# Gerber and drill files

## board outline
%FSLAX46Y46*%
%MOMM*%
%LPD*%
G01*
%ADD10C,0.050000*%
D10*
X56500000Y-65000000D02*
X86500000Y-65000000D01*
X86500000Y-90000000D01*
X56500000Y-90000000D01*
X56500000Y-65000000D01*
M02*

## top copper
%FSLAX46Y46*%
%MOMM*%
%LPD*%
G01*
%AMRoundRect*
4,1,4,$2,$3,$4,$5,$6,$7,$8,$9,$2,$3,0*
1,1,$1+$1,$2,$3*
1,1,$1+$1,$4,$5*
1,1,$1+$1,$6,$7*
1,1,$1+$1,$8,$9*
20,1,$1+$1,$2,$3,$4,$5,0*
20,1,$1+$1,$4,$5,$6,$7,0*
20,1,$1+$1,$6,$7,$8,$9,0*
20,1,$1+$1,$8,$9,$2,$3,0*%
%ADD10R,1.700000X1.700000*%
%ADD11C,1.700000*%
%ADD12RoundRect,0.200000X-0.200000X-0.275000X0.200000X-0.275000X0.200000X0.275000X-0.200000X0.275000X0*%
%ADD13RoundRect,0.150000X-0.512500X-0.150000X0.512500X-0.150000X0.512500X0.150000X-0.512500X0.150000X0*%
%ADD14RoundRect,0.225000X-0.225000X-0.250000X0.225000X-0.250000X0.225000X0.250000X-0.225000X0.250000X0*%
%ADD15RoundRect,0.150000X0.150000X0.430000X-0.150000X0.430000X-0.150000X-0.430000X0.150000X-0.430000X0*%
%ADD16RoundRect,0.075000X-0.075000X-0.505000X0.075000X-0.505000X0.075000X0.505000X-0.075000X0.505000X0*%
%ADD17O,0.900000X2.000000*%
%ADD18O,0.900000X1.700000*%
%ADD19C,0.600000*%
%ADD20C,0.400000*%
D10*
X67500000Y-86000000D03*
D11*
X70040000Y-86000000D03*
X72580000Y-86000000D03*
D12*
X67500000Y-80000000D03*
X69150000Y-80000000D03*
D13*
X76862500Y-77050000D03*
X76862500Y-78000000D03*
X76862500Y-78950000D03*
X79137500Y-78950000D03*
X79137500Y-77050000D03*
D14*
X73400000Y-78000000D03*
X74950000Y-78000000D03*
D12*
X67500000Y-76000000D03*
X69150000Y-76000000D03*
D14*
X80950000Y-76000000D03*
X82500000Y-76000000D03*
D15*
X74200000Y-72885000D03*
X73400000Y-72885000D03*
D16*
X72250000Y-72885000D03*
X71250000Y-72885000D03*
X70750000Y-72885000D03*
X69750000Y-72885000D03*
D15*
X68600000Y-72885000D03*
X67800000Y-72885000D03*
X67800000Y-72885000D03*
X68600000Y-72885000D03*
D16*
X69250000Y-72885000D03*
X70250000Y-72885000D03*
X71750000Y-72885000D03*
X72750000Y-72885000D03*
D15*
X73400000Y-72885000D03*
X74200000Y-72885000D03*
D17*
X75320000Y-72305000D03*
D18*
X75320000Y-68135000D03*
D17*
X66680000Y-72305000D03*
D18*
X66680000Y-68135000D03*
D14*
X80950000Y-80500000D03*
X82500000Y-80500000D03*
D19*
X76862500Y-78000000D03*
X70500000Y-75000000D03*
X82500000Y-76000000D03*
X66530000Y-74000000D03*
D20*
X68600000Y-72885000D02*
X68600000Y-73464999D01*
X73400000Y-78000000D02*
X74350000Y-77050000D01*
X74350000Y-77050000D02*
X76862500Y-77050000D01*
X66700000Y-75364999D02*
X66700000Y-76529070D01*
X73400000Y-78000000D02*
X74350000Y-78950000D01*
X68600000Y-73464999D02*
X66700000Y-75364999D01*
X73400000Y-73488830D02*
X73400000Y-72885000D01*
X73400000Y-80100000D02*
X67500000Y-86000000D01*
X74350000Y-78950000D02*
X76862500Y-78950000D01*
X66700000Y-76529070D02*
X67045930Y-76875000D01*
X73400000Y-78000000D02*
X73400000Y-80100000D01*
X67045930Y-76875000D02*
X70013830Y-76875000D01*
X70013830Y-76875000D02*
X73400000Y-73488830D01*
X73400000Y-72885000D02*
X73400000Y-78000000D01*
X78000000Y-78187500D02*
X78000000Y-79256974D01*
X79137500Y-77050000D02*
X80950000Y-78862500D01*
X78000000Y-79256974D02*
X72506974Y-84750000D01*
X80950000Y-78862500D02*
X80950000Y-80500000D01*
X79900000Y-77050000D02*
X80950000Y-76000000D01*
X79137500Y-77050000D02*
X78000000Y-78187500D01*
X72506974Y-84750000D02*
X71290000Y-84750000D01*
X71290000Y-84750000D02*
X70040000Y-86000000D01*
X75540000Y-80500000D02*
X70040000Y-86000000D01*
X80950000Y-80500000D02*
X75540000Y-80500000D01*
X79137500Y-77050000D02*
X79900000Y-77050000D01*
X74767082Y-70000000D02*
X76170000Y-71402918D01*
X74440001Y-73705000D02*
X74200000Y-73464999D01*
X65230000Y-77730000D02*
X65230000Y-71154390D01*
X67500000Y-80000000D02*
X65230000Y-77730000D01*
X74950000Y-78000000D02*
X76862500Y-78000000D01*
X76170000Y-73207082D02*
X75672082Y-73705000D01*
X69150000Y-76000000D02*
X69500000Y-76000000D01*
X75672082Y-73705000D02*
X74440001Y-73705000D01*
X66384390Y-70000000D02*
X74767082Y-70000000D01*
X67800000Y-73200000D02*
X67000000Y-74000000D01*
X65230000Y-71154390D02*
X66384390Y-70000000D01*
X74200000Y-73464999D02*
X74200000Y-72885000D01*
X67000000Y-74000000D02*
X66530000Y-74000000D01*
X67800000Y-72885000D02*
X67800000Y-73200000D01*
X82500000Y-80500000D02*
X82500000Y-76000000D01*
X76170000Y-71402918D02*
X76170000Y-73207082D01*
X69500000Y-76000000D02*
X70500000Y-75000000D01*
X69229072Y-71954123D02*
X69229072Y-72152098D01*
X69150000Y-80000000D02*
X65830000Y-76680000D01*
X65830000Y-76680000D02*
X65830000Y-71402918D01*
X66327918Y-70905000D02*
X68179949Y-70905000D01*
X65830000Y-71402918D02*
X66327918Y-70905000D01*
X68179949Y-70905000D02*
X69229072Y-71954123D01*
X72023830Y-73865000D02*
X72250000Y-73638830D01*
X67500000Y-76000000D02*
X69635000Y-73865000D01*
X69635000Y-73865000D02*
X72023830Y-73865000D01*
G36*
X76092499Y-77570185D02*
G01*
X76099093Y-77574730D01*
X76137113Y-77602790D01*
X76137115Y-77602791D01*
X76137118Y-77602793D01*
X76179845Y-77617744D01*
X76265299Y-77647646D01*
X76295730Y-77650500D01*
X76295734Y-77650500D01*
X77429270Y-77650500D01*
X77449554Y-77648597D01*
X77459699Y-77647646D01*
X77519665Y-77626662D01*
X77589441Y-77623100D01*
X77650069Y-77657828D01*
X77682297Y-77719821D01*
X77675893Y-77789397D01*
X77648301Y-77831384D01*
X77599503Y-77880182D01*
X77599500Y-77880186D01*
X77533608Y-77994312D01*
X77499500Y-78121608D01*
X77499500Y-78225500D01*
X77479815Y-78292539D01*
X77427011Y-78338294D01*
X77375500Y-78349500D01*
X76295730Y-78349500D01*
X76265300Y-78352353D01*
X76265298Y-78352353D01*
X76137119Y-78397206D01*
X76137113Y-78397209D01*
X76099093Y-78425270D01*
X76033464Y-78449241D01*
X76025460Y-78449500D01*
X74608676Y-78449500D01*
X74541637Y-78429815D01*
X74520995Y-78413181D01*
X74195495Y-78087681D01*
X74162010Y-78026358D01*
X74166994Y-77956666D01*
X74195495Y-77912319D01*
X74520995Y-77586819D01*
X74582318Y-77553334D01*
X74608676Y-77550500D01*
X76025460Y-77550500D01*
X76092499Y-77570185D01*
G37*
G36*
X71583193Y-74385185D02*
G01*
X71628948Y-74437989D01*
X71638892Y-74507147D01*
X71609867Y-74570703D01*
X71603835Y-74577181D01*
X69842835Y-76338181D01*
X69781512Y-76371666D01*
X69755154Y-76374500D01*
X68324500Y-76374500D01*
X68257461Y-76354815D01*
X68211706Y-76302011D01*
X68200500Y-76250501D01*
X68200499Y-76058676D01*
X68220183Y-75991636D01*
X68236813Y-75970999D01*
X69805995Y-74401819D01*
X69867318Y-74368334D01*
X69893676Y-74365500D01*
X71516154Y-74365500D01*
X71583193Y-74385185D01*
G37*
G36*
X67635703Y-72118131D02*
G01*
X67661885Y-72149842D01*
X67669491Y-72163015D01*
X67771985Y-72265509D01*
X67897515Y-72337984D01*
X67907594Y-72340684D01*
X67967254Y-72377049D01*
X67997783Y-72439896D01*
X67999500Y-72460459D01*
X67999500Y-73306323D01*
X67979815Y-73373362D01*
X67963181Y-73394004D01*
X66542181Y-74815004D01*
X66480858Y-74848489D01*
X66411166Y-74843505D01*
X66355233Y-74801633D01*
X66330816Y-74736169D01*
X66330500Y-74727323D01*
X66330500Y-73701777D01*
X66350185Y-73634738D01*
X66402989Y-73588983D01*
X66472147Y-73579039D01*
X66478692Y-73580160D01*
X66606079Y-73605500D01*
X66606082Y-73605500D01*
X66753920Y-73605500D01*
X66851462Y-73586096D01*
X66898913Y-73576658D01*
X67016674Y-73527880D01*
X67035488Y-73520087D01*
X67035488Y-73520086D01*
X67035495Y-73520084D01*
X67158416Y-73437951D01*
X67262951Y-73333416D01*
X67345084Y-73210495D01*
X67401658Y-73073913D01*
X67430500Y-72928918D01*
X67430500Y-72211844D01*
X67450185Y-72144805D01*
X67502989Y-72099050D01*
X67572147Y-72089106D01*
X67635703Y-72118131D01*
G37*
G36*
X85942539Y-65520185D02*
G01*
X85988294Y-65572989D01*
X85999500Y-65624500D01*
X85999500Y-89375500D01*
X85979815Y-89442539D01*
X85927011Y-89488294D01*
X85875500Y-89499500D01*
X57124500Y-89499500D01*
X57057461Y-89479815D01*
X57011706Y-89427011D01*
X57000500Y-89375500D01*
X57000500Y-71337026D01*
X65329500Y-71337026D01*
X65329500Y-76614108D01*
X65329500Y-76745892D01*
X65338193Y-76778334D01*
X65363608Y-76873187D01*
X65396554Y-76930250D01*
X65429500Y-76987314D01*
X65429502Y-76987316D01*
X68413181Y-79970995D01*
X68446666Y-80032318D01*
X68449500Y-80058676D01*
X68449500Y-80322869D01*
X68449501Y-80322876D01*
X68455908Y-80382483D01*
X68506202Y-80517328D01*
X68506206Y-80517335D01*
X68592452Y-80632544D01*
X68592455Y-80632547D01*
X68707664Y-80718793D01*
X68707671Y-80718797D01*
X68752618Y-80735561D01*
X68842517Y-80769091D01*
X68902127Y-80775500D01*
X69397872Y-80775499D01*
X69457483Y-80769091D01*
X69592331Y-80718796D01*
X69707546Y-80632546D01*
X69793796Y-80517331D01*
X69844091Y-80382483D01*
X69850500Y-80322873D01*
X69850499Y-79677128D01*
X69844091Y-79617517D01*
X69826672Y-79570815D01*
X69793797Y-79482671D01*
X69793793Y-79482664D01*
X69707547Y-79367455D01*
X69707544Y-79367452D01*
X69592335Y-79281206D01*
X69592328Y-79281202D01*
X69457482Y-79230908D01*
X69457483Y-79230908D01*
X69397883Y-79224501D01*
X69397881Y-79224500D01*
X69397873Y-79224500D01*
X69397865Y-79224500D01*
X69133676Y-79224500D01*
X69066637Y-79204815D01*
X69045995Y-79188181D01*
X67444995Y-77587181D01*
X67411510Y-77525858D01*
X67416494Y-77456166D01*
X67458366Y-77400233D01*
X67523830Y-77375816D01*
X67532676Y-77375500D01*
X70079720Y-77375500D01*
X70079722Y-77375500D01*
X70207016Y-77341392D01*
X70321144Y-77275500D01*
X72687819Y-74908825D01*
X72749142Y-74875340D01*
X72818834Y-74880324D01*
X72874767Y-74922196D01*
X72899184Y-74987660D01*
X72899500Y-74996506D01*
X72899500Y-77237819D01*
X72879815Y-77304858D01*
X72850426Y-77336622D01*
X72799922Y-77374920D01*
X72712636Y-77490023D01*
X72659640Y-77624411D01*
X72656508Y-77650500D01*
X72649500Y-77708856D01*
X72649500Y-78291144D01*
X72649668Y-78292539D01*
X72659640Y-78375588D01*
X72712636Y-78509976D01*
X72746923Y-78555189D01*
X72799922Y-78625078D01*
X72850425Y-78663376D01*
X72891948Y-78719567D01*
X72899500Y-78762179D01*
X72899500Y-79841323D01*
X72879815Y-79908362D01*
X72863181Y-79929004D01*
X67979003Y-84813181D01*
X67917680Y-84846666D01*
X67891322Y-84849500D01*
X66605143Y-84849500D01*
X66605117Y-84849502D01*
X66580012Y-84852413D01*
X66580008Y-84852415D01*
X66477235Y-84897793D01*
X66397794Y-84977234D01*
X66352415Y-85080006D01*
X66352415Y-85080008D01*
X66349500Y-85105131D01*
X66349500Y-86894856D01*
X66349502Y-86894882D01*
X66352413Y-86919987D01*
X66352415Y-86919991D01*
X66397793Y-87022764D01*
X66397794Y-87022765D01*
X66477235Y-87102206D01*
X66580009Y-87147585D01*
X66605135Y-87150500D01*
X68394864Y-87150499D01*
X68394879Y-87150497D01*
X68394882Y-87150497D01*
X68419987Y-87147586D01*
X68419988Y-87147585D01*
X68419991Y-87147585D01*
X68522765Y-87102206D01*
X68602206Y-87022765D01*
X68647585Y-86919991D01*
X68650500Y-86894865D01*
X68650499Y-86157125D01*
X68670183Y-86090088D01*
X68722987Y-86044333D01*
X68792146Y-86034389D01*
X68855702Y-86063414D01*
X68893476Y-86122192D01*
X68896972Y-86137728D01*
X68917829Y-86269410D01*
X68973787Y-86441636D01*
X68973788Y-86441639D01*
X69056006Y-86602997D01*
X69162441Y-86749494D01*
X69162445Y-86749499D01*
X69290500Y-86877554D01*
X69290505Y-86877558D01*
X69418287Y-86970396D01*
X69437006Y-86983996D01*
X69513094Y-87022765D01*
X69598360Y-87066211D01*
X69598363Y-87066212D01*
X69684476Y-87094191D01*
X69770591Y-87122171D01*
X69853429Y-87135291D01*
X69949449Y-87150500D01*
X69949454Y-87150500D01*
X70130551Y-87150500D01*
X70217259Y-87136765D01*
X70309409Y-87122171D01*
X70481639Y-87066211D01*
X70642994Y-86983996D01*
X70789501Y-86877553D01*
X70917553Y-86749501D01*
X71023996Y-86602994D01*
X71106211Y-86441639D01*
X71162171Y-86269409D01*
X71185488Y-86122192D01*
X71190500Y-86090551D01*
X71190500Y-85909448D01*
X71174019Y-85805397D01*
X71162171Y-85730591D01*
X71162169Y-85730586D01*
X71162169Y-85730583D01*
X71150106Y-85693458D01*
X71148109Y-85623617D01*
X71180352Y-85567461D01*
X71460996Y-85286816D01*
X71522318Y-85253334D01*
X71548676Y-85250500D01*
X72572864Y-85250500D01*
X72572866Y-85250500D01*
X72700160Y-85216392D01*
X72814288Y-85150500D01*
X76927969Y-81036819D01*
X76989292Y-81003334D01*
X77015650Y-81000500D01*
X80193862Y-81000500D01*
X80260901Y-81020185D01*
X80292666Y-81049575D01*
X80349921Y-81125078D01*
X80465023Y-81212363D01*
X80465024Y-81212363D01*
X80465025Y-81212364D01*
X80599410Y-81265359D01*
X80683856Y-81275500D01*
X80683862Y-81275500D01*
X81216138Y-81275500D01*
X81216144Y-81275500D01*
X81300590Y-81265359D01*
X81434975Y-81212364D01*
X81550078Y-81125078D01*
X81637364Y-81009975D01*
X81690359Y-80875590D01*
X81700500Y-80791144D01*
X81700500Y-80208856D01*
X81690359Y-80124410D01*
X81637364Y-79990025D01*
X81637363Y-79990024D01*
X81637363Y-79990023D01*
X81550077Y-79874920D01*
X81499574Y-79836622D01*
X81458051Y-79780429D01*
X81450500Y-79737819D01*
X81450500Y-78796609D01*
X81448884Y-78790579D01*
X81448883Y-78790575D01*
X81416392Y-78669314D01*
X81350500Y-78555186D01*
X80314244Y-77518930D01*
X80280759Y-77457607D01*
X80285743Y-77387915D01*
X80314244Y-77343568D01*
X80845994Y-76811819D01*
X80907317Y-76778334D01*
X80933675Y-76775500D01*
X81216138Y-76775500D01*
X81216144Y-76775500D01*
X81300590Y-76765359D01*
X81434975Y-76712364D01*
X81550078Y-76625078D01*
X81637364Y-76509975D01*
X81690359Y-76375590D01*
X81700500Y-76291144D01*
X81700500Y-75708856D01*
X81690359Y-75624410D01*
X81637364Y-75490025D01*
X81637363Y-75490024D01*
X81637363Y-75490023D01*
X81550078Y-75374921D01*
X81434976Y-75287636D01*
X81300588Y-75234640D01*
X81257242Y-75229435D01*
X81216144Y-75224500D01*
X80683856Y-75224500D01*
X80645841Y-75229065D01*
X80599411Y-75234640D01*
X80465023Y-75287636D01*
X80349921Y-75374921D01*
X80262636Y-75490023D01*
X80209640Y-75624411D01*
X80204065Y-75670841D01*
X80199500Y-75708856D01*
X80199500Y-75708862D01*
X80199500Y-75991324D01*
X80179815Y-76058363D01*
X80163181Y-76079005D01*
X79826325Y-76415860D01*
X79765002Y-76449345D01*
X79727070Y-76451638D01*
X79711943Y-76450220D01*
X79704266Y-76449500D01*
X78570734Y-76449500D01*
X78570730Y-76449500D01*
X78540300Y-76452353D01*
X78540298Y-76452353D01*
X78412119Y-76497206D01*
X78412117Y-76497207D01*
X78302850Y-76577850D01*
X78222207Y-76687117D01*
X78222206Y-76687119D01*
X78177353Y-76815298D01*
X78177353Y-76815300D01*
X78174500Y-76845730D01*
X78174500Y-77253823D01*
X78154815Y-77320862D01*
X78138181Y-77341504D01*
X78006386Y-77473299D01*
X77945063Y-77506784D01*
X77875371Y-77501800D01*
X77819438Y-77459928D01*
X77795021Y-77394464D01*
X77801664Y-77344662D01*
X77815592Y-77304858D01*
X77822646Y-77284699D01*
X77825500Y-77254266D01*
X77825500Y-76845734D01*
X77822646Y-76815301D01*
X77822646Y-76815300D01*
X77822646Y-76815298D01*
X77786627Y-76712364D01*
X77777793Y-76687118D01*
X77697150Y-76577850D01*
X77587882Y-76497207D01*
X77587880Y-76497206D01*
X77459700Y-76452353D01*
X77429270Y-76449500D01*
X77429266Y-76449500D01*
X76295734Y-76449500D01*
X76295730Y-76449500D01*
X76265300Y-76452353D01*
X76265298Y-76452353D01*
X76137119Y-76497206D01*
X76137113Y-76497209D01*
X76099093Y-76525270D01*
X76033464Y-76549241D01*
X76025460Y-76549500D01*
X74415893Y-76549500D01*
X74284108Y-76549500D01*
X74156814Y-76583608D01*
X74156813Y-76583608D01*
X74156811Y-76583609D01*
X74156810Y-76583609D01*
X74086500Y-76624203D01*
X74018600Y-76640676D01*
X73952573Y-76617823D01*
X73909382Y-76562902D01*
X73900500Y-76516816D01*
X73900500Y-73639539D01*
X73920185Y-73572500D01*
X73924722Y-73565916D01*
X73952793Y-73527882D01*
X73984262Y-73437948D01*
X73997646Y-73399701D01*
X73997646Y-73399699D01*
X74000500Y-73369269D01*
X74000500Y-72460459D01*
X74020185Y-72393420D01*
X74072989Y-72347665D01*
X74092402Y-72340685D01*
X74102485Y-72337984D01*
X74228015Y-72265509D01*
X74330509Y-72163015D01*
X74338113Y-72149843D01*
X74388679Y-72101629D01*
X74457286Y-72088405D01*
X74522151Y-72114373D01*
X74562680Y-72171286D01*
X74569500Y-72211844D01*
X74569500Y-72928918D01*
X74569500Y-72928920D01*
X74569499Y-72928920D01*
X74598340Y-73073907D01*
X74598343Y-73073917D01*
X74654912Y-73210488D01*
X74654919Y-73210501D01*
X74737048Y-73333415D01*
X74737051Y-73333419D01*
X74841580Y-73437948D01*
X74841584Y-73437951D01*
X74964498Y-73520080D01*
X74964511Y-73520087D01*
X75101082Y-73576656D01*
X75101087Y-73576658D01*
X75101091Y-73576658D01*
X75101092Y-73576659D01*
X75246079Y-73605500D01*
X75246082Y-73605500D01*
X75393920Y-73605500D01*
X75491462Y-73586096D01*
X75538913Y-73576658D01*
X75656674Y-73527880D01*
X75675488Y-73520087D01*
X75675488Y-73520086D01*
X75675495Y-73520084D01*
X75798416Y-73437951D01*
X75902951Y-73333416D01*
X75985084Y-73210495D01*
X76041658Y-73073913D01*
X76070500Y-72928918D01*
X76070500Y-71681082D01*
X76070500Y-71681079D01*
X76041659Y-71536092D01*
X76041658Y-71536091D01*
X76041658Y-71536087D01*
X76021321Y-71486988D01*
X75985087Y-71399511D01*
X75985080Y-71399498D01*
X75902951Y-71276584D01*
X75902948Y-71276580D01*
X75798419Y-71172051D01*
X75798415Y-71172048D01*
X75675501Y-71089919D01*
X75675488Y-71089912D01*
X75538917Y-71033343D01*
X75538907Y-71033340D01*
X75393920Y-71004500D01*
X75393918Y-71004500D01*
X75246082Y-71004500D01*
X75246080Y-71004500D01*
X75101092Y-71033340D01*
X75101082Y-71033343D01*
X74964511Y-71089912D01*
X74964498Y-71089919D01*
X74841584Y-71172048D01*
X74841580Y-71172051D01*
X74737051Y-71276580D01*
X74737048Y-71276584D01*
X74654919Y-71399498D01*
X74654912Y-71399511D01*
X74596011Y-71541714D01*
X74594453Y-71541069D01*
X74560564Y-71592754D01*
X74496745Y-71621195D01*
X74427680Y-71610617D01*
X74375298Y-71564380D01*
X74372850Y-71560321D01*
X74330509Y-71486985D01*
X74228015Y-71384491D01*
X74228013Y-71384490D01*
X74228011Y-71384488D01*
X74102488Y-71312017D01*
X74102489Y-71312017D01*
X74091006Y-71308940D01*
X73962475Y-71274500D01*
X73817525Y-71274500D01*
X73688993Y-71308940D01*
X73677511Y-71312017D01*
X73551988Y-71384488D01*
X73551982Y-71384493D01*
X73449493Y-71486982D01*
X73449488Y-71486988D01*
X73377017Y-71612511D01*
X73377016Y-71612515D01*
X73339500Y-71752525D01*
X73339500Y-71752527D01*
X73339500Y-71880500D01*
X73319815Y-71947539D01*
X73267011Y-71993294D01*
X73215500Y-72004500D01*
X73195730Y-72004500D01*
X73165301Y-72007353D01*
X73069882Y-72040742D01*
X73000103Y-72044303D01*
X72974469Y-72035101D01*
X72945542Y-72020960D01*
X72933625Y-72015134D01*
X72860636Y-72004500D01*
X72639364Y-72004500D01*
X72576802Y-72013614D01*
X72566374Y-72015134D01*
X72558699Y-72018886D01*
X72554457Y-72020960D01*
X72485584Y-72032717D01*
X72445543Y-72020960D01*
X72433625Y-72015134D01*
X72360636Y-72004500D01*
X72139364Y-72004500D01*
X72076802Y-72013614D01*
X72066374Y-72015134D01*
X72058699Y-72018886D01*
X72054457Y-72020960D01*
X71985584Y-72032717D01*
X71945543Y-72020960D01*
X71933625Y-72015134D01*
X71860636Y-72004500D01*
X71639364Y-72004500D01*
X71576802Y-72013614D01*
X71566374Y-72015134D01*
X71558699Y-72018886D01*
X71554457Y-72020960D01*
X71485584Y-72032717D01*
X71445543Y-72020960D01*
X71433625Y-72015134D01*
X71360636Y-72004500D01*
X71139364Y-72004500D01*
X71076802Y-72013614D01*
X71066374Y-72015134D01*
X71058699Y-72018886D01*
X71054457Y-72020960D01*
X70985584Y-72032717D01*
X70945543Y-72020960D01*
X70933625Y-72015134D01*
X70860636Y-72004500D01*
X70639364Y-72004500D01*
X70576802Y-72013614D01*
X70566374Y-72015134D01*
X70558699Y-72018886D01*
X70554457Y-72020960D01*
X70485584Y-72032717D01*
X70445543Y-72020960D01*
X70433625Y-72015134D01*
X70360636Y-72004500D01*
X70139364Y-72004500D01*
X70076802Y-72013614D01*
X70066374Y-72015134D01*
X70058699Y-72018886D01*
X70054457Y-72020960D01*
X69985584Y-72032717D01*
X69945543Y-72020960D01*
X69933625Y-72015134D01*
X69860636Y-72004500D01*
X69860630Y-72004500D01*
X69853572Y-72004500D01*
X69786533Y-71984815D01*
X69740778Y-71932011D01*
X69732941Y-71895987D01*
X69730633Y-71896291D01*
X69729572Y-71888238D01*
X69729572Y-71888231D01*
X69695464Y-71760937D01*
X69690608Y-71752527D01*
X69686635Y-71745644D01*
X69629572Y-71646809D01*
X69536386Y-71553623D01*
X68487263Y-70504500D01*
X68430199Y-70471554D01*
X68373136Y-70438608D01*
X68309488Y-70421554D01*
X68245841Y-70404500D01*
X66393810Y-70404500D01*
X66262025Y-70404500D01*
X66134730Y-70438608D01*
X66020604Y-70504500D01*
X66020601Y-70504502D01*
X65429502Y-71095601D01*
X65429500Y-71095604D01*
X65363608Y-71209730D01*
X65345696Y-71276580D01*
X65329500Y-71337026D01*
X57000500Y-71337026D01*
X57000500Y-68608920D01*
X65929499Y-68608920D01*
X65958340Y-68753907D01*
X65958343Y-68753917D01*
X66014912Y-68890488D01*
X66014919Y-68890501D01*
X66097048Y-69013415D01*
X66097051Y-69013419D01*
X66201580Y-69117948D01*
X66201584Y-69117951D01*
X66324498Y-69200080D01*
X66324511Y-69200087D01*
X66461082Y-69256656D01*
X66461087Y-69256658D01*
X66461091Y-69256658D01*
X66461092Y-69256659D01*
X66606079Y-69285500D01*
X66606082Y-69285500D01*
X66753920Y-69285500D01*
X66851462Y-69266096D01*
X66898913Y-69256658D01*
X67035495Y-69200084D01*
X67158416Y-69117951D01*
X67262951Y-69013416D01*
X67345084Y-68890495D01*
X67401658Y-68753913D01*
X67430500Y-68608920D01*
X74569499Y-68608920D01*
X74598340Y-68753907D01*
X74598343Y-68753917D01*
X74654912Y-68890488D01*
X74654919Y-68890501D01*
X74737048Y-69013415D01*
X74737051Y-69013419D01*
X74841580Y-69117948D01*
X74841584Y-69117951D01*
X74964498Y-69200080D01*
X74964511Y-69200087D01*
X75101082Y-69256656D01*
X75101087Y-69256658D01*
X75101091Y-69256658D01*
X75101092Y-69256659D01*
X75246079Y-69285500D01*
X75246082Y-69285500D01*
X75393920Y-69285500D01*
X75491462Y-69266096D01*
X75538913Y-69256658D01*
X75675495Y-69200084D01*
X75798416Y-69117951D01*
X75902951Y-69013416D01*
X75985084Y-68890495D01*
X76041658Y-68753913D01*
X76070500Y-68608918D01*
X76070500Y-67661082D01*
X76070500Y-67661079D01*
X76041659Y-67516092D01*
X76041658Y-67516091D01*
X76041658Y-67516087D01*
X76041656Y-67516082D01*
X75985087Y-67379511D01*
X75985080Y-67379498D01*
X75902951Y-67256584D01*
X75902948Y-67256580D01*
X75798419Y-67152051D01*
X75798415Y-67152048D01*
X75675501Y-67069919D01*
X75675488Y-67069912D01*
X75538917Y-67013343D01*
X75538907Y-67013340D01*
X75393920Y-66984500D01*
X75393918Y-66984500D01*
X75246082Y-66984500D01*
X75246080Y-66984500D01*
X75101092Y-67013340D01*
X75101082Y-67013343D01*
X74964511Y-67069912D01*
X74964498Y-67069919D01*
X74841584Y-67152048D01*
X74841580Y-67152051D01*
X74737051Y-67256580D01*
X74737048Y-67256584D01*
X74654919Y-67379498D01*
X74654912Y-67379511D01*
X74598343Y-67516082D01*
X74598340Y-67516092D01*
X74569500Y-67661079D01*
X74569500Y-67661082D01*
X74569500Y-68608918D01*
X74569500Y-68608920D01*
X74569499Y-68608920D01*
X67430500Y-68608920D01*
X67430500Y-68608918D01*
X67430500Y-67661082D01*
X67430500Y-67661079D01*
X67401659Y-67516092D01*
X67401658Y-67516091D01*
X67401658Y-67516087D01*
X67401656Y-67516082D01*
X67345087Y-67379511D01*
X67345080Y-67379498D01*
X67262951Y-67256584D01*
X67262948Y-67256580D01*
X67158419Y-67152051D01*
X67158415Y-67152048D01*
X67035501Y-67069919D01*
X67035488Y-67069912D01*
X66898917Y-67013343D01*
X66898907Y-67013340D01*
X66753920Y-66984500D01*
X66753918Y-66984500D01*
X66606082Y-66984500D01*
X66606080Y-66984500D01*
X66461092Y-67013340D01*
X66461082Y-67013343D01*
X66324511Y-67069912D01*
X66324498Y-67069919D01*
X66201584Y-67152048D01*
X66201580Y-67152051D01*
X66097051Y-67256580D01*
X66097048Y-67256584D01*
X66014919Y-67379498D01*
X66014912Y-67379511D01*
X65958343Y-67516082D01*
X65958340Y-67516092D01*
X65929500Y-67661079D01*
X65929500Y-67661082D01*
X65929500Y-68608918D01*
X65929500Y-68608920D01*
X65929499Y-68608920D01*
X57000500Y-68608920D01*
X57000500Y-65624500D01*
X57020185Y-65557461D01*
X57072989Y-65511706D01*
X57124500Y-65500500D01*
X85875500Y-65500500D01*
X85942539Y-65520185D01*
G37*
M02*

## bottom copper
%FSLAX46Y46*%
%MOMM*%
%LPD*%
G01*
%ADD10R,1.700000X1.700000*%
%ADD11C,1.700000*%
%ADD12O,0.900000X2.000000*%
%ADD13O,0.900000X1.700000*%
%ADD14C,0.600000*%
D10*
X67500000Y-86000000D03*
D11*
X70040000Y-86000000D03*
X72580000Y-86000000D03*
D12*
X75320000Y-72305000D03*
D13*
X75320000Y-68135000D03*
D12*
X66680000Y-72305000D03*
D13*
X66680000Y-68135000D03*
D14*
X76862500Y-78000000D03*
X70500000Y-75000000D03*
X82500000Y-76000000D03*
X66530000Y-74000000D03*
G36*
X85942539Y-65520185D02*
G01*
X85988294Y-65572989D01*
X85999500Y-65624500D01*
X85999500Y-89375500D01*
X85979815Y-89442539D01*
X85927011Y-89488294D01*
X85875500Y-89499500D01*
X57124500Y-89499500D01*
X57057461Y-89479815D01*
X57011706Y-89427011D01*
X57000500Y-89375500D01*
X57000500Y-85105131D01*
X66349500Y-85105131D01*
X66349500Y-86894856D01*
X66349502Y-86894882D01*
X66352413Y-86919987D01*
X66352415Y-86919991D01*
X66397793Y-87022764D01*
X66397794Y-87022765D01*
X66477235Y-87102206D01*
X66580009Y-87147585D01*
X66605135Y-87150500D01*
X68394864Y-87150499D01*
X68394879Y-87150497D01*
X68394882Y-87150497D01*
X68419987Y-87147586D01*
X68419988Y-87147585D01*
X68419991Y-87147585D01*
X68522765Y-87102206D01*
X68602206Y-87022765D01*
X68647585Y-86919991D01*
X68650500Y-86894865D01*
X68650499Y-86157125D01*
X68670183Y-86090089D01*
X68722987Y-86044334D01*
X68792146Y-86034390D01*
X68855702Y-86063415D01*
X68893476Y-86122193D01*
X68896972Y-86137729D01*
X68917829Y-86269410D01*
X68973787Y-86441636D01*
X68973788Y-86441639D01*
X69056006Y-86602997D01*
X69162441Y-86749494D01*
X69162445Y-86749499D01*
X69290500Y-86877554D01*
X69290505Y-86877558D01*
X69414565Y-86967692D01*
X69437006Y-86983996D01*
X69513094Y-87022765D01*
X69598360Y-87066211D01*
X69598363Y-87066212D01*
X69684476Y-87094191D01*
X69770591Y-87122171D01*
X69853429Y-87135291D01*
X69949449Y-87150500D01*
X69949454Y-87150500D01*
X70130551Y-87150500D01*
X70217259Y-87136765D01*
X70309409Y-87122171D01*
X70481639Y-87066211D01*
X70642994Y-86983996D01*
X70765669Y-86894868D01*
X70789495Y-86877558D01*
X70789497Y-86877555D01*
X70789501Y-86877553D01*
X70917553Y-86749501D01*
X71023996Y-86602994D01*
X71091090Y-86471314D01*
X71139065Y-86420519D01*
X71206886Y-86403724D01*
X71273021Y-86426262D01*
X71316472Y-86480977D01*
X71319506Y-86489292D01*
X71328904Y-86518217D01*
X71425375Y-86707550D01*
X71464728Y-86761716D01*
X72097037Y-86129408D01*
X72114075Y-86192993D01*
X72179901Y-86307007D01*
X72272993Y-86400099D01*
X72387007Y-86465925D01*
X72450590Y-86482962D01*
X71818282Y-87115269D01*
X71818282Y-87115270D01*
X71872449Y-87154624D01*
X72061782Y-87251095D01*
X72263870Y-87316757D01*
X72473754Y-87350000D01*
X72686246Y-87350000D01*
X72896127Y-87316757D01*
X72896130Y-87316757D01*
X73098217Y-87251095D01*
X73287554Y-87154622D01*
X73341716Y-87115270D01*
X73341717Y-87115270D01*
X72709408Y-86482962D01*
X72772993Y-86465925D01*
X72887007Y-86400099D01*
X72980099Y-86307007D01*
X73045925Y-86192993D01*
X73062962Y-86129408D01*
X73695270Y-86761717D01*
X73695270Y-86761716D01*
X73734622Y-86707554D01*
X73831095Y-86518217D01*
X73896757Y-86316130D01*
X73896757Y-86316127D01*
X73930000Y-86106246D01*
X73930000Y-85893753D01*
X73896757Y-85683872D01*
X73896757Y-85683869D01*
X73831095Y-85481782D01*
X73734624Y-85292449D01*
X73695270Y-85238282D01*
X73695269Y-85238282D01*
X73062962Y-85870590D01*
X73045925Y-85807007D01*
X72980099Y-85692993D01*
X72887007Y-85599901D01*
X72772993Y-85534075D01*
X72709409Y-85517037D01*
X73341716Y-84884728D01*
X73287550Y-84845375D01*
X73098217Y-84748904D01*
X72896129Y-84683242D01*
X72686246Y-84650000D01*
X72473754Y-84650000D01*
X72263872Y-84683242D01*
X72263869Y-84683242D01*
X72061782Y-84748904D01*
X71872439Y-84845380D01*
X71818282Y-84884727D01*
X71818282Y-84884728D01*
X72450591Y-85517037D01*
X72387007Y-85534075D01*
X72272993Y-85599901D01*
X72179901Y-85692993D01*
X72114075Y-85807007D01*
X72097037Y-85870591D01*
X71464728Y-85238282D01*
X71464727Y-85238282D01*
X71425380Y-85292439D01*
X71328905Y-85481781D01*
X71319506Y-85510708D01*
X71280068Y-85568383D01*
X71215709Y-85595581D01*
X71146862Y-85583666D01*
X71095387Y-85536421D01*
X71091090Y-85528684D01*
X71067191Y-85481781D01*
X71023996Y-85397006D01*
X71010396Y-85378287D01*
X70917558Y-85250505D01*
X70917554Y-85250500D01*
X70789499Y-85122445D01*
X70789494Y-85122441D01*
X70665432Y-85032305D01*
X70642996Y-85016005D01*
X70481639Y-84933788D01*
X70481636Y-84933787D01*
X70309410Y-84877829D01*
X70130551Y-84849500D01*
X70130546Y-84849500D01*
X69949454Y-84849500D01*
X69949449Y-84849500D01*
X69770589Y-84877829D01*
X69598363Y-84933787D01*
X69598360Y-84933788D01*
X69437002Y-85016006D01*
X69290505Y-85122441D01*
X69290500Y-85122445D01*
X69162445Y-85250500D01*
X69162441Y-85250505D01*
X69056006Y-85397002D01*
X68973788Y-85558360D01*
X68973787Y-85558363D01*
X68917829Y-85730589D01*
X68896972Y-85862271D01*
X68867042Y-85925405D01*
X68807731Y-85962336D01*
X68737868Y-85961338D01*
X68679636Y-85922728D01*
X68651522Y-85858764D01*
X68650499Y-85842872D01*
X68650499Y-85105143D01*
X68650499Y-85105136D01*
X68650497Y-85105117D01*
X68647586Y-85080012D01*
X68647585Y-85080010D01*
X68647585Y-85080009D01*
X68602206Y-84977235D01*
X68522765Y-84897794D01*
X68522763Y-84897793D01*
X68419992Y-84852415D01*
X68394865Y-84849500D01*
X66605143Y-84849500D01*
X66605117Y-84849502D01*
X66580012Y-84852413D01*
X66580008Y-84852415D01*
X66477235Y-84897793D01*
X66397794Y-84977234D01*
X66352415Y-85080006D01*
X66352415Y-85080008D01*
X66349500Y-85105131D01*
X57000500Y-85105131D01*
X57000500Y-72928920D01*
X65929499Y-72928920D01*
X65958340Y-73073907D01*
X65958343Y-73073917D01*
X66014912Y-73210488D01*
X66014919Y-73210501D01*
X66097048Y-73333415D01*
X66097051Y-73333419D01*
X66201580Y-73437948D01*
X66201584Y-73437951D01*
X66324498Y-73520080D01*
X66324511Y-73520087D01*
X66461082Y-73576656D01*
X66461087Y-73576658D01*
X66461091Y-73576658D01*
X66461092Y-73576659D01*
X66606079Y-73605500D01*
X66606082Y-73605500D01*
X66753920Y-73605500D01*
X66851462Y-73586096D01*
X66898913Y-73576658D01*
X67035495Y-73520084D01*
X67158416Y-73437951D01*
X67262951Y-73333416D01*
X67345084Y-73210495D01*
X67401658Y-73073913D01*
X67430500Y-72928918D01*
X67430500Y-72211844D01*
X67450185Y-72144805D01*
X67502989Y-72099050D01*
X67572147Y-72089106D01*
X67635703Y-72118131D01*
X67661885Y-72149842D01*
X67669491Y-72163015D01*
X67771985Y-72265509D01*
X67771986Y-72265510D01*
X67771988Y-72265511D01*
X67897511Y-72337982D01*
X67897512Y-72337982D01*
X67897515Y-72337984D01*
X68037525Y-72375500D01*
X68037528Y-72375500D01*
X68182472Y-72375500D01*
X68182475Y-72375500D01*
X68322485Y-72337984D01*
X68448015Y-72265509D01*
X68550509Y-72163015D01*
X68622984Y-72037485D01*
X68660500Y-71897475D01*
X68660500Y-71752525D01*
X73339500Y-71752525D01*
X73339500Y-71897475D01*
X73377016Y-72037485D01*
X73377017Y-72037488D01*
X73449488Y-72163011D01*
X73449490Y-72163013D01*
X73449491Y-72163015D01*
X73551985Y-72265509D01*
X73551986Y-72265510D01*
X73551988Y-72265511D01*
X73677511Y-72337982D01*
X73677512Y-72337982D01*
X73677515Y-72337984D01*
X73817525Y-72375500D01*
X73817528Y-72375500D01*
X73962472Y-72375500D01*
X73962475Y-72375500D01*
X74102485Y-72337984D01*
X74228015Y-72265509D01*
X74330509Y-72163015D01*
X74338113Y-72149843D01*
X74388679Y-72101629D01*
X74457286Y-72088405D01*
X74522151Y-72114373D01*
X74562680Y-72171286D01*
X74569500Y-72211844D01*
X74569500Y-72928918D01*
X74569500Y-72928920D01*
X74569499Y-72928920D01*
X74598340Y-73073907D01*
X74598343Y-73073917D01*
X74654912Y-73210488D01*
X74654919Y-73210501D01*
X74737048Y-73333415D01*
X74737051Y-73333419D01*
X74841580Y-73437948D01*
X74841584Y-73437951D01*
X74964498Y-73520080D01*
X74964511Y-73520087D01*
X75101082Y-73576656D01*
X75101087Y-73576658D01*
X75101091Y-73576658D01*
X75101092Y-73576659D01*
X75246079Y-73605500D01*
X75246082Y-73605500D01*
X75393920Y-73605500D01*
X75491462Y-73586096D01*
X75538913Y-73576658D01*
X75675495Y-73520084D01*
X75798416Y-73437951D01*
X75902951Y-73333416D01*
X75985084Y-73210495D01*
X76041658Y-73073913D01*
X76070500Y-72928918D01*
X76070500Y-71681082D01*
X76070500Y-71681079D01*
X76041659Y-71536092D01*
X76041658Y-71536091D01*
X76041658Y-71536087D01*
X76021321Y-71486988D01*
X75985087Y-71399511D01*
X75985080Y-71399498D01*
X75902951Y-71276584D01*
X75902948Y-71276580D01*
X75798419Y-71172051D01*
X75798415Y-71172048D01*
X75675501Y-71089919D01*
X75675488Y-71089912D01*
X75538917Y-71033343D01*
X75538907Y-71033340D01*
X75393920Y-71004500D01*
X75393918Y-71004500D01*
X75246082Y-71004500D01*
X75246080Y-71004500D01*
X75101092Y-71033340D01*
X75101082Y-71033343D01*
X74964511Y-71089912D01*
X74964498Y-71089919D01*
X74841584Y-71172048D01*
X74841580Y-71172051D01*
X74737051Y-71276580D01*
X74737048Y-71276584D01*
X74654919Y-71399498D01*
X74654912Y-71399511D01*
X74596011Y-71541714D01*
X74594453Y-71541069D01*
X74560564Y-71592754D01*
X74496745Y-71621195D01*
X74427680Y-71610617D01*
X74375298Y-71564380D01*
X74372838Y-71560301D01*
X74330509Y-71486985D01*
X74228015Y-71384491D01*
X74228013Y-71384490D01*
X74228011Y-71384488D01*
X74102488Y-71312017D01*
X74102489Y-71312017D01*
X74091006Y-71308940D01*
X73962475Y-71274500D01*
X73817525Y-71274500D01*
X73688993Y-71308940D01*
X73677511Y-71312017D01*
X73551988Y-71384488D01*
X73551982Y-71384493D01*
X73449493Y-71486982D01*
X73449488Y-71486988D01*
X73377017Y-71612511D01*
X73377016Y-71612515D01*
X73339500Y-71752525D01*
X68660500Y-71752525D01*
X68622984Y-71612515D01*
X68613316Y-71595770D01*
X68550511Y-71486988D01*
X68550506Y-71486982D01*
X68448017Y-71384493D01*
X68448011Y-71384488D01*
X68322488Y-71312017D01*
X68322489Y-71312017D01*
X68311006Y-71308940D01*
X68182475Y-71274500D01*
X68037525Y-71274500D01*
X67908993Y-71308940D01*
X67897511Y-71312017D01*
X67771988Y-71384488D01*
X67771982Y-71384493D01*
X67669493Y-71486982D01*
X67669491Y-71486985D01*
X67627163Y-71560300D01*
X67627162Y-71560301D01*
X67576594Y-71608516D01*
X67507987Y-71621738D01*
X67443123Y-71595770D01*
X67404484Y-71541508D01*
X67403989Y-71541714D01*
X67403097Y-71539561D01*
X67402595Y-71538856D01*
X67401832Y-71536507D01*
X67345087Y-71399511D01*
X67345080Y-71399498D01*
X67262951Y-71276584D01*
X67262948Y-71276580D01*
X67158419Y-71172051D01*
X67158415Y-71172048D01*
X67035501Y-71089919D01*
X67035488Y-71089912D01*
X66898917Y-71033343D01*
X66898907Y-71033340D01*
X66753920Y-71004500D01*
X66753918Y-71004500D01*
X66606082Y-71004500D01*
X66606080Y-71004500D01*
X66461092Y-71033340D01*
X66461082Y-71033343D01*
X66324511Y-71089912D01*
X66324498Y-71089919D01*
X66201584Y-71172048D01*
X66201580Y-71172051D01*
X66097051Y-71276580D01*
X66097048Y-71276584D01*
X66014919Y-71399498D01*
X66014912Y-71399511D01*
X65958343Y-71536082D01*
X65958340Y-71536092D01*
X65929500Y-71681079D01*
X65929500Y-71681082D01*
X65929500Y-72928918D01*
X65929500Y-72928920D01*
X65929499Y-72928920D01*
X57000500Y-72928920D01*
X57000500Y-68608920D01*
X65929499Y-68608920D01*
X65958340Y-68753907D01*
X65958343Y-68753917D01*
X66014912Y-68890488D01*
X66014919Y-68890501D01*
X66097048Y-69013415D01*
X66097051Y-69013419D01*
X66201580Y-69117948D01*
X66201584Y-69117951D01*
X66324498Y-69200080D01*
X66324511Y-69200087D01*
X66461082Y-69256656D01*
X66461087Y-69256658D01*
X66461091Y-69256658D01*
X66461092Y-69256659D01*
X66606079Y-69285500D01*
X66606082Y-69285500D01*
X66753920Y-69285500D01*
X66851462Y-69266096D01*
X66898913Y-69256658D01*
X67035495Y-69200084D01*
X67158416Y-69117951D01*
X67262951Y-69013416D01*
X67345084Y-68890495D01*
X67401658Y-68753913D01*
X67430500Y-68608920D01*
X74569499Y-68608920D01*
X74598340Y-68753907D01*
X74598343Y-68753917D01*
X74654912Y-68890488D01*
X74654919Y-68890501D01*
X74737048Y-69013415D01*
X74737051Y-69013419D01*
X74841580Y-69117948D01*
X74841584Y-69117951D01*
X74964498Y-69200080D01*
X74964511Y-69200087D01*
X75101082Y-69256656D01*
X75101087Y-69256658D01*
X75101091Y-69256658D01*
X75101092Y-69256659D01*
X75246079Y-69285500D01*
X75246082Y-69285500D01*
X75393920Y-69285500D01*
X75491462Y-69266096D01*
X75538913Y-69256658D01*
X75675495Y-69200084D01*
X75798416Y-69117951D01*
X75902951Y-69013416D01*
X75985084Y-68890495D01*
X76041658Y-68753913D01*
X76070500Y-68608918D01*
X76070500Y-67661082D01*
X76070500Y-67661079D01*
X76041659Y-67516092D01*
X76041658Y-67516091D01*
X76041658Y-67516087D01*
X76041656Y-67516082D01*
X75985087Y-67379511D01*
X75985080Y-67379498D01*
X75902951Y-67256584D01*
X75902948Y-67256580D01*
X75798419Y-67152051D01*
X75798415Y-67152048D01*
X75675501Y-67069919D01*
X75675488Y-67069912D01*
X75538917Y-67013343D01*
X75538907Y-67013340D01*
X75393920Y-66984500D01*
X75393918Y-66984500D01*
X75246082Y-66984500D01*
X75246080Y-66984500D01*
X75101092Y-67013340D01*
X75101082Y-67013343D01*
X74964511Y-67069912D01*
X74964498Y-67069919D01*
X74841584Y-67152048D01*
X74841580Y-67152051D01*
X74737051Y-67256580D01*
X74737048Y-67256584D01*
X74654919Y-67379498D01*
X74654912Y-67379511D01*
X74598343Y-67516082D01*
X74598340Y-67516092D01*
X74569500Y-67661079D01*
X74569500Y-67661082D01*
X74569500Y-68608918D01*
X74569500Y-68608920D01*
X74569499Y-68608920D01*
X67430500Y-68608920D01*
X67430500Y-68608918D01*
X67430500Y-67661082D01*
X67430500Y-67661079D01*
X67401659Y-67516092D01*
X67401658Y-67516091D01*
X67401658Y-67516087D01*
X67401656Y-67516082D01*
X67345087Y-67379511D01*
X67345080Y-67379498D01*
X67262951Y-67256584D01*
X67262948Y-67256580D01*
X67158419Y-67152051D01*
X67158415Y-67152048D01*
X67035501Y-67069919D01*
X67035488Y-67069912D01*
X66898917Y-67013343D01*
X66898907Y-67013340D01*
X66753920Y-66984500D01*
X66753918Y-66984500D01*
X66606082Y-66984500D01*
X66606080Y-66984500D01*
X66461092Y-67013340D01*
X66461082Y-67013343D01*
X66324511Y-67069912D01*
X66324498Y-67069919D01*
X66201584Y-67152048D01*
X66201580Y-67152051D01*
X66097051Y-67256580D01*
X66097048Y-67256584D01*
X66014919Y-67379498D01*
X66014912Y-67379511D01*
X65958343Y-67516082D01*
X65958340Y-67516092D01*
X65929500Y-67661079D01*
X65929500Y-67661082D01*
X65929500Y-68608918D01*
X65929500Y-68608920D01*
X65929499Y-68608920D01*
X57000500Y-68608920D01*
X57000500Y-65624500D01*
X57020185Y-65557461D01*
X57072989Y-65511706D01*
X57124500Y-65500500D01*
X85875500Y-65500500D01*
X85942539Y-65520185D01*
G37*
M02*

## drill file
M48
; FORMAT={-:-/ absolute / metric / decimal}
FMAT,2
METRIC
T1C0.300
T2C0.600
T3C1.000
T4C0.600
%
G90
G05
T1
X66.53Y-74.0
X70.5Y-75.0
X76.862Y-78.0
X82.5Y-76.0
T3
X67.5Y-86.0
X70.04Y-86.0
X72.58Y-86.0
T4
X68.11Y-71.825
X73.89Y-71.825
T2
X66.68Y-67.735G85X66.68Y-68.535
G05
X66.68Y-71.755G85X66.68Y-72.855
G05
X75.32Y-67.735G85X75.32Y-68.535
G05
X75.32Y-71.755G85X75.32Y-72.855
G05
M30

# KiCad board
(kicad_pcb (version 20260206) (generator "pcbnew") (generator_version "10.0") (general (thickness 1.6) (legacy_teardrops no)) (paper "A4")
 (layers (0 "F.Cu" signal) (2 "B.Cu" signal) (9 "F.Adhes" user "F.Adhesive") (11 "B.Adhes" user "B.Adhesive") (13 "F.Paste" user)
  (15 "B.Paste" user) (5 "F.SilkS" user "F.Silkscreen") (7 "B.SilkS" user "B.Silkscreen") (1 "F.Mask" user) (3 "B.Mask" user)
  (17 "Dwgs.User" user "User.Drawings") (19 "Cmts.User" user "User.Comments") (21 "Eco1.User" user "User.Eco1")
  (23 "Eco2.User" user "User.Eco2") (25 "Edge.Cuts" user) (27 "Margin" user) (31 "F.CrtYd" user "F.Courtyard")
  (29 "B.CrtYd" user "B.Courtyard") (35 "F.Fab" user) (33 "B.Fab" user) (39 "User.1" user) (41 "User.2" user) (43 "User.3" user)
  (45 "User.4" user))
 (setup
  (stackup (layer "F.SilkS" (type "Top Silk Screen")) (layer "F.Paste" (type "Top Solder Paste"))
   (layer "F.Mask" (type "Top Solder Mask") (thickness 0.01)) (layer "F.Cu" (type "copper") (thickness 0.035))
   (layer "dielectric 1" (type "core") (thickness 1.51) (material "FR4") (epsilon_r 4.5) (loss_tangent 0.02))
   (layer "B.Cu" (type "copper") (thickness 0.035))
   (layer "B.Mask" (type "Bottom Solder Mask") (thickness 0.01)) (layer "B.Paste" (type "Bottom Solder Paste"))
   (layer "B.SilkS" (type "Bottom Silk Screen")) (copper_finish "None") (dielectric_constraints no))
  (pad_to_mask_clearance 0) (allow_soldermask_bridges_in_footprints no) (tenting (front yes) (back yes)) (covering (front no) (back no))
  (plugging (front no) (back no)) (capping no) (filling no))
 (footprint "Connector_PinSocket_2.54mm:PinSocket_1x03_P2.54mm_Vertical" (layer "F.Cu") (at 67.5 86 90)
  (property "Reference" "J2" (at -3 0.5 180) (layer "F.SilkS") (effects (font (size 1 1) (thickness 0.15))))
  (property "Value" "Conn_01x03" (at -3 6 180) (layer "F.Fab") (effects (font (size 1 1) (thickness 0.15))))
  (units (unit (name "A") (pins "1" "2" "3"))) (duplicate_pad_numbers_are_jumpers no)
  (pad "1" thru_hole rect (at 0 0 90) (size 1.7 1.7) (drill 1) (layers "*.Cu" "*.Mask") (remove_unused_layers no) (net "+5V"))
  (pad "2" thru_hole circle (at 0 2.54 90) (size 1.7 1.7) (drill 1) (layers "*.Cu" "*.Mask") (remove_unused_layers no) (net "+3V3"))
  (pad "3" thru_hole circle (at 0 5.08 90) (size 1.7 1.7) (drill 1) (layers "*.Cu" "*.Mask") (remove_unused_layers no) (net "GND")))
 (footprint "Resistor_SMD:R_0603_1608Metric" (layer "F.Cu") (at 68.325 80)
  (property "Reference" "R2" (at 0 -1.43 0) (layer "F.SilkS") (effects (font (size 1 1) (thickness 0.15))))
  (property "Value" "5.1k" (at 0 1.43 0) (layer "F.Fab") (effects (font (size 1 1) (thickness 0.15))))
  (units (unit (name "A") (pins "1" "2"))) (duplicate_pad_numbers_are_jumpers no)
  (pad "1" smd roundrect (at -0.825 0) (size 0.8 0.95) (layers "F.Cu" "F.Mask" "F.Paste") (roundrect_rratio 0.25) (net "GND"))
  (pad "2" smd roundrect (at 0.825 0) (size 0.8 0.95) (layers "F.Cu" "F.Mask" "F.Paste") (roundrect_rratio 0.25) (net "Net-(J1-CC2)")))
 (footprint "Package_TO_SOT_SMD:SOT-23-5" (layer "F.Cu") (at 78 78)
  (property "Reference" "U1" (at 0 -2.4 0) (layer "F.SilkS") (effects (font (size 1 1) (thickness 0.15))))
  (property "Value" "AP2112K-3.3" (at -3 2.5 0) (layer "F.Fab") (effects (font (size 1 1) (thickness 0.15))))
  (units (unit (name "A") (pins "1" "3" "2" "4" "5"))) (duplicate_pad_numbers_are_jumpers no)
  (pad "1" smd roundrect (at -1.1375 -0.95) (size 1.325 0.6) (layers "F.Cu" "F.Mask" "F.Paste") (roundrect_rratio 0.25) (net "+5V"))
  (pad "2" smd roundrect (at -1.1375 0) (size 1.325 0.6) (layers "F.Cu" "F.Mask" "F.Paste") (roundrect_rratio 0.25) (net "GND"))
  (pad "3" smd roundrect (at -1.1375 0.95) (size 1.325 0.6) (layers "F.Cu" "F.Mask" "F.Paste") (roundrect_rratio 0.25) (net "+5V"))
  (pad "4" smd roundrect (at 1.1375 0.95) (size 1.325 0.6) (layers "F.Cu" "F.Mask" "F.Paste") (roundrect_rratio 0.25)
   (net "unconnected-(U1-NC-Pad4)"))
  (pad "5" smd roundrect (at 1.1375 -0.95) (size 1.325 0.6) (layers "F.Cu" "F.Mask" "F.Paste") (roundrect_rratio 0.25) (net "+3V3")))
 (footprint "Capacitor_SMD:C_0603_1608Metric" (layer "F.Cu") (at 74.175 78)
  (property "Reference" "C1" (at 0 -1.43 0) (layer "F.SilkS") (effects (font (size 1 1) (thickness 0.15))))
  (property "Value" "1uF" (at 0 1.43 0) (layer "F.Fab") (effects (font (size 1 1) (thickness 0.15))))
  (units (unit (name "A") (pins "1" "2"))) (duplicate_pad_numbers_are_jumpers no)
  (pad "1" smd roundrect (at -0.775 0) (size 0.9 0.95) (layers "F.Cu" "F.Mask" "F.Paste") (roundrect_rratio 0.25) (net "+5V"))
  (pad "2" smd roundrect (at 0.775 0) (size 0.9 0.95) (layers "F.Cu" "F.Mask" "F.Paste") (roundrect_rratio 0.25) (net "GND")))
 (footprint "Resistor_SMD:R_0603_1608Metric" (layer "F.Cu") (at 68.325 76)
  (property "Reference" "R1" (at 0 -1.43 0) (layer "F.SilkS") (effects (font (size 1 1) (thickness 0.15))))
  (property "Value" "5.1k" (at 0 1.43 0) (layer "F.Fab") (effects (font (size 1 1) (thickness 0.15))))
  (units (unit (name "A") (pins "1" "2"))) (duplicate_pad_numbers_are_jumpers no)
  (pad "1" smd roundrect (at -0.825 0) (size 0.8 0.95) (layers "F.Cu" "F.Mask" "F.Paste") (roundrect_rratio 0.25) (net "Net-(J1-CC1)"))
  (pad "2" smd roundrect (at 0.825 0) (size 0.8 0.95) (layers "F.Cu" "F.Mask" "F.Paste") (roundrect_rratio 0.25) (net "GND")))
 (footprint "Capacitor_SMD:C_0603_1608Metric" (layer "F.Cu") (at 81.725 76)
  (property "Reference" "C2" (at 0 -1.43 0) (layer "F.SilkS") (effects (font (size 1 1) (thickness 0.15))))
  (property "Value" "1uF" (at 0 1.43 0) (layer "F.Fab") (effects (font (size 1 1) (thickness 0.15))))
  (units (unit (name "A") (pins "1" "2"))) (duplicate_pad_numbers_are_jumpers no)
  (pad "1" smd roundrect (at -0.775 0) (size 0.9 0.95) (layers "F.Cu" "F.Mask" "F.Paste") (roundrect_rratio 0.25) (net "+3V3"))
  (pad "2" smd roundrect (at 0.775 0) (size 0.9 0.95) (layers "F.Cu" "F.Mask" "F.Paste") (roundrect_rratio 0.25) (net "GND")))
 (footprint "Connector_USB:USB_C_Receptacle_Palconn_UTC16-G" (layer "F.Cu") (at 71 70.375 180)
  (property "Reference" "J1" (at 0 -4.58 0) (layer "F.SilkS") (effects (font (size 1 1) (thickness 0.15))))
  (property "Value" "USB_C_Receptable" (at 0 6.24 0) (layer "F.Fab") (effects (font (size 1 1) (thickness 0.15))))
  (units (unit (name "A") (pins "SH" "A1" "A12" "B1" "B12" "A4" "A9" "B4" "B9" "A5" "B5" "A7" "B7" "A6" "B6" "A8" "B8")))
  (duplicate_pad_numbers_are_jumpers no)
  (pad "" np_thru_hole circle (at -2.89 -1.45) (size 0.6 0.6) (drill 0.6) (layers "*.Cu" "*.Mask"))
  (pad "" np_thru_hole circle (at 2.89 -1.45) (size 0.6 0.6) (drill 0.6) (layers "*.Cu" "*.Mask"))
  (pad "A1" smd roundrect (at -3.2 -2.51 180) (size 0.6 1.16) (layers "F.Cu" "F.Mask" "F.Paste") (roundrect_rratio 0.25) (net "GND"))
  (pad "A4" smd roundrect (at -2.4 -2.51 180) (size 0.6 1.16) (layers "F.Cu" "F.Mask" "F.Paste") (roundrect_rratio 0.25) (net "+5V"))
  (pad "A5" smd roundrect (at -1.25 -2.51) (size 0.3 1.16) (layers "F.Cu" "F.Mask" "F.Paste") (roundrect_rratio 0.25) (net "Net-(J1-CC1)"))
  (pad "A6" smd roundrect (at -0.25 -2.51) (size 0.3 1.16) (layers "F.Cu" "F.Mask" "F.Paste") (roundrect_rratio 0.25)
   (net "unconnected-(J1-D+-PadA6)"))
  (pad "A7" smd roundrect (at 0.25 -2.51) (size 0.3 1.16) (layers "F.Cu" "F.Mask" "F.Paste") (roundrect_rratio 0.25)
   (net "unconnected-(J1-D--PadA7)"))
  (pad "A8" smd roundrect (at 1.25 -2.51) (size 0.3 1.16) (layers "F.Cu" "F.Mask" "F.Paste") (roundrect_rratio 0.25)
   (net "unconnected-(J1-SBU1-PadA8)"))
  (pad "A9" smd roundrect (at 2.4 -2.51 180) (size 0.6 1.16) (layers "F.Cu" "F.Mask" "F.Paste") (roundrect_rratio 0.25) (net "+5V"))
  (pad "A12" smd roundrect (at 3.2 -2.51 180) (size 0.6 1.16) (layers "F.Cu" "F.Mask" "F.Paste") (roundrect_rratio 0.25) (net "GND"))
  (pad "B1" smd roundrect (at 3.2 -2.51 180) (size 0.6 1.16) (layers "F.Cu" "F.Mask" "F.Paste") (roundrect_rratio 0.25) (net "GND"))
  (pad "B4" smd roundrect (at 2.4 -2.51 180) (size 0.6 1.16) (layers "F.Cu" "F.Mask" "F.Paste") (roundrect_rratio 0.25) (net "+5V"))
  (pad "B5" smd roundrect (at 1.75 -2.51) (size 0.3 1.16) (layers "F.Cu" "F.Mask" "F.Paste") (roundrect_rratio 0.25) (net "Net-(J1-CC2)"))
  (pad "B6" smd roundrect (at 0.75 -2.51) (size 0.3 1.16) (layers "F.Cu" "F.Mask" "F.Paste") (roundrect_rratio 0.25)
   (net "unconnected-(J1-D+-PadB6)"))
  (pad "B7" smd roundrect (at -0.75 -2.51) (size 0.3 1.16) (layers "F.Cu" "F.Mask" "F.Paste") (roundrect_rratio 0.25)
   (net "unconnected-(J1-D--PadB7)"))
  (pad "B8" smd roundrect (at -1.75 -2.51) (size 0.3 1.16) (layers "F.Cu" "F.Mask" "F.Paste") (roundrect_rratio 0.25)
   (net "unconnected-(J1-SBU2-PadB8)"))
  (pad "B9" smd roundrect (at -2.4 -2.51 180) (size 0.6 1.16) (layers "F.Cu" "F.Mask" "F.Paste") (roundrect_rratio 0.25) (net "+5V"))
  (pad "B12" smd roundrect (at -3.2 -2.51 180) (size 0.6 1.16) (layers "F.Cu" "F.Mask" "F.Paste") (roundrect_rratio 0.25) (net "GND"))
  (pad "SH" thru_hole oval (at -4.32 -1.93 270) (size 2 0.9) (drill oval 1.7 0.6) (layers "*.Cu" "*.Mask") (remove_unused_layers no)
   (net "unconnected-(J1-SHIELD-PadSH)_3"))
  (pad "SH" thru_hole oval (at -4.32 2.24 270) (size 1.7 0.9) (drill oval 1.4 0.6) (layers "*.Cu" "*.Mask") (remove_unused_layers no)
   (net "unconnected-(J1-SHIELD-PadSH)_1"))
  (pad "SH" thru_hole oval (at 4.32 -1.93 270) (size 2 0.9) (drill oval 1.7 0.6) (layers "*.Cu" "*.Mask") (remove_unused_layers no)
   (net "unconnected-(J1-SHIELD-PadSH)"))
  (pad "SH" thru_hole oval (at 4.32 2.24 270) (size 1.7 0.9) (drill oval 1.4 0.6) (layers "*.Cu" "*.Mask") (remove_unused_layers no)
   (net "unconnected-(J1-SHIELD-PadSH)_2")))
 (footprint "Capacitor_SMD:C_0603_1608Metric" (layer "F.Cu") (at 81.725 80.5)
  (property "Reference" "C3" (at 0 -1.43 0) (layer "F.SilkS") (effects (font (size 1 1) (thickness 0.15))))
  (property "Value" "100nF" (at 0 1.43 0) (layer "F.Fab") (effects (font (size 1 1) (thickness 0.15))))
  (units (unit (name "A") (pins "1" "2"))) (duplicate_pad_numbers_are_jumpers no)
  (pad "1" smd roundrect (at -0.775 0) (size 0.9 0.95) (layers "F.Cu" "F.Mask" "F.Paste") (roundrect_rratio 0.25) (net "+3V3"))
  (pad "2" smd roundrect (at 0.775 0) (size 0.9 0.95) (layers "F.Cu" "F.Mask" "F.Paste") (roundrect_rratio 0.25) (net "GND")))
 (gr_rect (start 56.5 65) (end 86.5 90) (stroke (width 0.05) (type default)) (fill no) (layer "Edge.Cuts"))
 (segment (start 68.6 72.885) (end 68.6 73.464999) (width 0.4) (layer "F.Cu") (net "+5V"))
 (segment (start 73.4 78) (end 74.35 77.05) (width 0.4) (layer "F.Cu") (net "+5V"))
 (segment (start 74.35 77.05) (end 76.8625 77.05) (width 0.4) (layer "F.Cu") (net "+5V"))
 (segment (start 66.7 75.364999) (end 66.7 76.52907) (width 0.4) (layer "F.Cu") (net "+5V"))
 (segment (start 73.4 78) (end 74.35 78.95) (width 0.4) (layer "F.Cu") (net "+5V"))
 (segment (start 68.6 73.464999) (end 66.7 75.364999) (width 0.4) (layer "F.Cu") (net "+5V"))
 (segment (start 73.4 73.48883) (end 73.4 72.885) (width 0.4) (layer "F.Cu") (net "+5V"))
 (segment (start 73.4 80.1) (end 67.5 86) (width 0.4) (layer "F.Cu") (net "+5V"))
 (segment (start 74.35 78.95) (end 76.8625 78.95) (width 0.4) (layer "F.Cu") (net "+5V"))
 (segment (start 66.7 76.52907) (end 67.04593 76.875) (width 0.4) (layer "F.Cu") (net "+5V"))
 (segment (start 73.4 78) (end 73.4 80.1) (width 0.4) (layer "F.Cu") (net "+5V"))
 (segment (start 67.04593 76.875) (end 70.01383 76.875) (width 0.4) (layer "F.Cu") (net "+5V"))
 (segment (start 70.01383 76.875) (end 73.4 73.48883) (width 0.4) (layer "F.Cu") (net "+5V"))
 (segment (start 73.4 72.885) (end 73.4 78) (width 0.4) (layer "F.Cu") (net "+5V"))
 (segment (start 78 78.1875) (end 78 79.256974) (width 0.4) (layer "F.Cu") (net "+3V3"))
 (segment (start 79.1375 77.05) (end 80.95 78.8625) (width 0.4) (layer "F.Cu") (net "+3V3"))
 (segment (start 78 79.256974) (end 72.506974 84.75) (width 0.4) (layer "F.Cu") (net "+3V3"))
 (segment (start 80.95 78.8625) (end 80.95 80.5) (width 0.4) (layer "F.Cu") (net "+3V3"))
 (segment (start 79.9 77.05) (end 80.95 76) (width 0.4) (layer "F.Cu") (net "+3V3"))
 (segment (start 79.1375 77.05) (end 78 78.1875) (width 0.4) (layer "F.Cu") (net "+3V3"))
 (segment (start 72.506974 84.75) (end 71.29 84.75) (width 0.4) (layer "F.Cu") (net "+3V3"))
 (segment (start 71.29 84.75) (end 70.04 86) (width 0.4) (layer "F.Cu") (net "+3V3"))
 (segment (start 75.54 80.5) (end 70.04 86) (width 0.4) (layer "F.Cu") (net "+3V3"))
 (segment (start 80.95 80.5) (end 75.54 80.5) (width 0.4) (layer "F.Cu") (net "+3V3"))
 (segment (start 79.1375 77.05) (end 79.9 77.05) (width 0.4) (layer "F.Cu") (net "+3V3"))
 (segment (start 74.767082 70) (end 76.17 71.402918) (width 0.4) (layer "F.Cu") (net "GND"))
 (segment (start 74.440001 73.705) (end 74.2 73.464999) (width 0.4) (layer "F.Cu") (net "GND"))
 (segment (start 65.23 77.73) (end 65.23 71.15439) (width 0.4) (layer "F.Cu") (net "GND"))
 (segment (start 67.5 80) (end 65.23 77.73) (width 0.4) (layer "F.Cu") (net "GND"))
 (segment (start 74.95 78) (end 76.8625 78) (width 0.4) (layer "F.Cu") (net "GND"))
 (segment (start 76.17 73.207082) (end 75.672082 73.705) (width 0.4) (layer "F.Cu") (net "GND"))
 (segment (start 69.15 76) (end 69.5 76) (width 0.4) (layer "F.Cu") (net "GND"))
 (segment (start 75.672082 73.705) (end 74.440001 73.705) (width 0.4) (layer "F.Cu") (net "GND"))
 (segment (start 66.38439 70) (end 74.767082 70) (width 0.4) (layer "F.Cu") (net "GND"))
 (segment (start 67.8 73.2) (end 67 74) (width 0.4) (layer "F.Cu") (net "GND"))
 (segment (start 65.23 71.15439) (end 66.38439 70) (width 0.4) (layer "F.Cu") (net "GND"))
 (segment (start 74.2 73.464999) (end 74.2 72.885) (width 0.4) (layer "F.Cu") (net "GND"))
 (segment (start 67 74) (end 66.53 74) (width 0.4) (layer "F.Cu") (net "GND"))
 (segment (start 67.8 72.885) (end 67.8 73.2) (width 0.4) (layer "F.Cu") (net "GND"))
 (segment (start 82.5 80.5) (end 82.5 76) (width 0.4) (layer "F.Cu") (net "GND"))
 (segment (start 76.17 71.402918) (end 76.17 73.207082) (width 0.4) (layer "F.Cu") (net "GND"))
 (segment (start 69.5 76) (end 70.5 75) (width 0.4) (layer "F.Cu") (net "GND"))
 (via (at 76.8625 78) (size 0.6) (drill 0.3) (layers "F.Cu" "B.Cu") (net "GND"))
 (via (at 70.5 75) (size 0.6) (drill 0.3) (layers "F.Cu" "B.Cu") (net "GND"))
 (via (at 82.5 76) (size 0.6) (drill 0.3) (layers "F.Cu" "B.Cu") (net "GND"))
 (via (at 66.53 74) (size 0.6) (drill 0.3) (layers "F.Cu" "B.Cu") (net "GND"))
 (segment (start 69.229072 71.954123) (end 69.229072 72.152098) (width 0.4) (layer "F.Cu") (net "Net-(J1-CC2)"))
 (segment (start 69.15 80) (end 65.83 76.68) (width 0.4) (layer "F.Cu") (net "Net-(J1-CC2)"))
 (segment (start 65.83 76.68) (end 65.83 71.402918) (width 0.4) (layer "F.Cu") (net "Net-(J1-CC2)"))
 (segment (start 66.327918 70.905) (end 68.179949 70.905) (width 0.4) (layer "F.Cu") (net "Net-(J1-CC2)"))
 (segment (start 65.83 71.402918) (end 66.327918 70.905) (width 0.4) (layer "F.Cu") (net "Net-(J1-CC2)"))
 (segment (start 68.179949 70.905) (end 69.229072 71.954123) (width 0.4) (layer "F.Cu") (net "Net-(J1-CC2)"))
 (segment (start 72.02383 73.865) (end 72.25 73.63883) (width 0.4) (layer "F.Cu") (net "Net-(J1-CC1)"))
 (segment (start 67.5 76) (end 69.635 73.865) (width 0.4) (layer "F.Cu") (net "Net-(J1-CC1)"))
 (segment (start 69.635 73.865) (end 72.02383 73.865) (width 0.4) (layer "F.Cu") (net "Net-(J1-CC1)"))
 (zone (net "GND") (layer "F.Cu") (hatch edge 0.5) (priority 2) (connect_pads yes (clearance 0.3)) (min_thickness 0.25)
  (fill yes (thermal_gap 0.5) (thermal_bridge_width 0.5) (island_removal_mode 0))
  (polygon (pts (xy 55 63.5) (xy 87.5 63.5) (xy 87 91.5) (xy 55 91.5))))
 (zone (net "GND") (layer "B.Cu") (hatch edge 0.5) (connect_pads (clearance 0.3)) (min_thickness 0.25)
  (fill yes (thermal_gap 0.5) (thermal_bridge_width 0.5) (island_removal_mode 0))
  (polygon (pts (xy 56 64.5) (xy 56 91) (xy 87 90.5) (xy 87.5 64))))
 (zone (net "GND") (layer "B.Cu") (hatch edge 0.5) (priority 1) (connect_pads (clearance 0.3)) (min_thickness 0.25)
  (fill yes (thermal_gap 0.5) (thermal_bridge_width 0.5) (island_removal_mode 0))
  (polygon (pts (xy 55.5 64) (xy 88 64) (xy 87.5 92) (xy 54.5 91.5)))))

